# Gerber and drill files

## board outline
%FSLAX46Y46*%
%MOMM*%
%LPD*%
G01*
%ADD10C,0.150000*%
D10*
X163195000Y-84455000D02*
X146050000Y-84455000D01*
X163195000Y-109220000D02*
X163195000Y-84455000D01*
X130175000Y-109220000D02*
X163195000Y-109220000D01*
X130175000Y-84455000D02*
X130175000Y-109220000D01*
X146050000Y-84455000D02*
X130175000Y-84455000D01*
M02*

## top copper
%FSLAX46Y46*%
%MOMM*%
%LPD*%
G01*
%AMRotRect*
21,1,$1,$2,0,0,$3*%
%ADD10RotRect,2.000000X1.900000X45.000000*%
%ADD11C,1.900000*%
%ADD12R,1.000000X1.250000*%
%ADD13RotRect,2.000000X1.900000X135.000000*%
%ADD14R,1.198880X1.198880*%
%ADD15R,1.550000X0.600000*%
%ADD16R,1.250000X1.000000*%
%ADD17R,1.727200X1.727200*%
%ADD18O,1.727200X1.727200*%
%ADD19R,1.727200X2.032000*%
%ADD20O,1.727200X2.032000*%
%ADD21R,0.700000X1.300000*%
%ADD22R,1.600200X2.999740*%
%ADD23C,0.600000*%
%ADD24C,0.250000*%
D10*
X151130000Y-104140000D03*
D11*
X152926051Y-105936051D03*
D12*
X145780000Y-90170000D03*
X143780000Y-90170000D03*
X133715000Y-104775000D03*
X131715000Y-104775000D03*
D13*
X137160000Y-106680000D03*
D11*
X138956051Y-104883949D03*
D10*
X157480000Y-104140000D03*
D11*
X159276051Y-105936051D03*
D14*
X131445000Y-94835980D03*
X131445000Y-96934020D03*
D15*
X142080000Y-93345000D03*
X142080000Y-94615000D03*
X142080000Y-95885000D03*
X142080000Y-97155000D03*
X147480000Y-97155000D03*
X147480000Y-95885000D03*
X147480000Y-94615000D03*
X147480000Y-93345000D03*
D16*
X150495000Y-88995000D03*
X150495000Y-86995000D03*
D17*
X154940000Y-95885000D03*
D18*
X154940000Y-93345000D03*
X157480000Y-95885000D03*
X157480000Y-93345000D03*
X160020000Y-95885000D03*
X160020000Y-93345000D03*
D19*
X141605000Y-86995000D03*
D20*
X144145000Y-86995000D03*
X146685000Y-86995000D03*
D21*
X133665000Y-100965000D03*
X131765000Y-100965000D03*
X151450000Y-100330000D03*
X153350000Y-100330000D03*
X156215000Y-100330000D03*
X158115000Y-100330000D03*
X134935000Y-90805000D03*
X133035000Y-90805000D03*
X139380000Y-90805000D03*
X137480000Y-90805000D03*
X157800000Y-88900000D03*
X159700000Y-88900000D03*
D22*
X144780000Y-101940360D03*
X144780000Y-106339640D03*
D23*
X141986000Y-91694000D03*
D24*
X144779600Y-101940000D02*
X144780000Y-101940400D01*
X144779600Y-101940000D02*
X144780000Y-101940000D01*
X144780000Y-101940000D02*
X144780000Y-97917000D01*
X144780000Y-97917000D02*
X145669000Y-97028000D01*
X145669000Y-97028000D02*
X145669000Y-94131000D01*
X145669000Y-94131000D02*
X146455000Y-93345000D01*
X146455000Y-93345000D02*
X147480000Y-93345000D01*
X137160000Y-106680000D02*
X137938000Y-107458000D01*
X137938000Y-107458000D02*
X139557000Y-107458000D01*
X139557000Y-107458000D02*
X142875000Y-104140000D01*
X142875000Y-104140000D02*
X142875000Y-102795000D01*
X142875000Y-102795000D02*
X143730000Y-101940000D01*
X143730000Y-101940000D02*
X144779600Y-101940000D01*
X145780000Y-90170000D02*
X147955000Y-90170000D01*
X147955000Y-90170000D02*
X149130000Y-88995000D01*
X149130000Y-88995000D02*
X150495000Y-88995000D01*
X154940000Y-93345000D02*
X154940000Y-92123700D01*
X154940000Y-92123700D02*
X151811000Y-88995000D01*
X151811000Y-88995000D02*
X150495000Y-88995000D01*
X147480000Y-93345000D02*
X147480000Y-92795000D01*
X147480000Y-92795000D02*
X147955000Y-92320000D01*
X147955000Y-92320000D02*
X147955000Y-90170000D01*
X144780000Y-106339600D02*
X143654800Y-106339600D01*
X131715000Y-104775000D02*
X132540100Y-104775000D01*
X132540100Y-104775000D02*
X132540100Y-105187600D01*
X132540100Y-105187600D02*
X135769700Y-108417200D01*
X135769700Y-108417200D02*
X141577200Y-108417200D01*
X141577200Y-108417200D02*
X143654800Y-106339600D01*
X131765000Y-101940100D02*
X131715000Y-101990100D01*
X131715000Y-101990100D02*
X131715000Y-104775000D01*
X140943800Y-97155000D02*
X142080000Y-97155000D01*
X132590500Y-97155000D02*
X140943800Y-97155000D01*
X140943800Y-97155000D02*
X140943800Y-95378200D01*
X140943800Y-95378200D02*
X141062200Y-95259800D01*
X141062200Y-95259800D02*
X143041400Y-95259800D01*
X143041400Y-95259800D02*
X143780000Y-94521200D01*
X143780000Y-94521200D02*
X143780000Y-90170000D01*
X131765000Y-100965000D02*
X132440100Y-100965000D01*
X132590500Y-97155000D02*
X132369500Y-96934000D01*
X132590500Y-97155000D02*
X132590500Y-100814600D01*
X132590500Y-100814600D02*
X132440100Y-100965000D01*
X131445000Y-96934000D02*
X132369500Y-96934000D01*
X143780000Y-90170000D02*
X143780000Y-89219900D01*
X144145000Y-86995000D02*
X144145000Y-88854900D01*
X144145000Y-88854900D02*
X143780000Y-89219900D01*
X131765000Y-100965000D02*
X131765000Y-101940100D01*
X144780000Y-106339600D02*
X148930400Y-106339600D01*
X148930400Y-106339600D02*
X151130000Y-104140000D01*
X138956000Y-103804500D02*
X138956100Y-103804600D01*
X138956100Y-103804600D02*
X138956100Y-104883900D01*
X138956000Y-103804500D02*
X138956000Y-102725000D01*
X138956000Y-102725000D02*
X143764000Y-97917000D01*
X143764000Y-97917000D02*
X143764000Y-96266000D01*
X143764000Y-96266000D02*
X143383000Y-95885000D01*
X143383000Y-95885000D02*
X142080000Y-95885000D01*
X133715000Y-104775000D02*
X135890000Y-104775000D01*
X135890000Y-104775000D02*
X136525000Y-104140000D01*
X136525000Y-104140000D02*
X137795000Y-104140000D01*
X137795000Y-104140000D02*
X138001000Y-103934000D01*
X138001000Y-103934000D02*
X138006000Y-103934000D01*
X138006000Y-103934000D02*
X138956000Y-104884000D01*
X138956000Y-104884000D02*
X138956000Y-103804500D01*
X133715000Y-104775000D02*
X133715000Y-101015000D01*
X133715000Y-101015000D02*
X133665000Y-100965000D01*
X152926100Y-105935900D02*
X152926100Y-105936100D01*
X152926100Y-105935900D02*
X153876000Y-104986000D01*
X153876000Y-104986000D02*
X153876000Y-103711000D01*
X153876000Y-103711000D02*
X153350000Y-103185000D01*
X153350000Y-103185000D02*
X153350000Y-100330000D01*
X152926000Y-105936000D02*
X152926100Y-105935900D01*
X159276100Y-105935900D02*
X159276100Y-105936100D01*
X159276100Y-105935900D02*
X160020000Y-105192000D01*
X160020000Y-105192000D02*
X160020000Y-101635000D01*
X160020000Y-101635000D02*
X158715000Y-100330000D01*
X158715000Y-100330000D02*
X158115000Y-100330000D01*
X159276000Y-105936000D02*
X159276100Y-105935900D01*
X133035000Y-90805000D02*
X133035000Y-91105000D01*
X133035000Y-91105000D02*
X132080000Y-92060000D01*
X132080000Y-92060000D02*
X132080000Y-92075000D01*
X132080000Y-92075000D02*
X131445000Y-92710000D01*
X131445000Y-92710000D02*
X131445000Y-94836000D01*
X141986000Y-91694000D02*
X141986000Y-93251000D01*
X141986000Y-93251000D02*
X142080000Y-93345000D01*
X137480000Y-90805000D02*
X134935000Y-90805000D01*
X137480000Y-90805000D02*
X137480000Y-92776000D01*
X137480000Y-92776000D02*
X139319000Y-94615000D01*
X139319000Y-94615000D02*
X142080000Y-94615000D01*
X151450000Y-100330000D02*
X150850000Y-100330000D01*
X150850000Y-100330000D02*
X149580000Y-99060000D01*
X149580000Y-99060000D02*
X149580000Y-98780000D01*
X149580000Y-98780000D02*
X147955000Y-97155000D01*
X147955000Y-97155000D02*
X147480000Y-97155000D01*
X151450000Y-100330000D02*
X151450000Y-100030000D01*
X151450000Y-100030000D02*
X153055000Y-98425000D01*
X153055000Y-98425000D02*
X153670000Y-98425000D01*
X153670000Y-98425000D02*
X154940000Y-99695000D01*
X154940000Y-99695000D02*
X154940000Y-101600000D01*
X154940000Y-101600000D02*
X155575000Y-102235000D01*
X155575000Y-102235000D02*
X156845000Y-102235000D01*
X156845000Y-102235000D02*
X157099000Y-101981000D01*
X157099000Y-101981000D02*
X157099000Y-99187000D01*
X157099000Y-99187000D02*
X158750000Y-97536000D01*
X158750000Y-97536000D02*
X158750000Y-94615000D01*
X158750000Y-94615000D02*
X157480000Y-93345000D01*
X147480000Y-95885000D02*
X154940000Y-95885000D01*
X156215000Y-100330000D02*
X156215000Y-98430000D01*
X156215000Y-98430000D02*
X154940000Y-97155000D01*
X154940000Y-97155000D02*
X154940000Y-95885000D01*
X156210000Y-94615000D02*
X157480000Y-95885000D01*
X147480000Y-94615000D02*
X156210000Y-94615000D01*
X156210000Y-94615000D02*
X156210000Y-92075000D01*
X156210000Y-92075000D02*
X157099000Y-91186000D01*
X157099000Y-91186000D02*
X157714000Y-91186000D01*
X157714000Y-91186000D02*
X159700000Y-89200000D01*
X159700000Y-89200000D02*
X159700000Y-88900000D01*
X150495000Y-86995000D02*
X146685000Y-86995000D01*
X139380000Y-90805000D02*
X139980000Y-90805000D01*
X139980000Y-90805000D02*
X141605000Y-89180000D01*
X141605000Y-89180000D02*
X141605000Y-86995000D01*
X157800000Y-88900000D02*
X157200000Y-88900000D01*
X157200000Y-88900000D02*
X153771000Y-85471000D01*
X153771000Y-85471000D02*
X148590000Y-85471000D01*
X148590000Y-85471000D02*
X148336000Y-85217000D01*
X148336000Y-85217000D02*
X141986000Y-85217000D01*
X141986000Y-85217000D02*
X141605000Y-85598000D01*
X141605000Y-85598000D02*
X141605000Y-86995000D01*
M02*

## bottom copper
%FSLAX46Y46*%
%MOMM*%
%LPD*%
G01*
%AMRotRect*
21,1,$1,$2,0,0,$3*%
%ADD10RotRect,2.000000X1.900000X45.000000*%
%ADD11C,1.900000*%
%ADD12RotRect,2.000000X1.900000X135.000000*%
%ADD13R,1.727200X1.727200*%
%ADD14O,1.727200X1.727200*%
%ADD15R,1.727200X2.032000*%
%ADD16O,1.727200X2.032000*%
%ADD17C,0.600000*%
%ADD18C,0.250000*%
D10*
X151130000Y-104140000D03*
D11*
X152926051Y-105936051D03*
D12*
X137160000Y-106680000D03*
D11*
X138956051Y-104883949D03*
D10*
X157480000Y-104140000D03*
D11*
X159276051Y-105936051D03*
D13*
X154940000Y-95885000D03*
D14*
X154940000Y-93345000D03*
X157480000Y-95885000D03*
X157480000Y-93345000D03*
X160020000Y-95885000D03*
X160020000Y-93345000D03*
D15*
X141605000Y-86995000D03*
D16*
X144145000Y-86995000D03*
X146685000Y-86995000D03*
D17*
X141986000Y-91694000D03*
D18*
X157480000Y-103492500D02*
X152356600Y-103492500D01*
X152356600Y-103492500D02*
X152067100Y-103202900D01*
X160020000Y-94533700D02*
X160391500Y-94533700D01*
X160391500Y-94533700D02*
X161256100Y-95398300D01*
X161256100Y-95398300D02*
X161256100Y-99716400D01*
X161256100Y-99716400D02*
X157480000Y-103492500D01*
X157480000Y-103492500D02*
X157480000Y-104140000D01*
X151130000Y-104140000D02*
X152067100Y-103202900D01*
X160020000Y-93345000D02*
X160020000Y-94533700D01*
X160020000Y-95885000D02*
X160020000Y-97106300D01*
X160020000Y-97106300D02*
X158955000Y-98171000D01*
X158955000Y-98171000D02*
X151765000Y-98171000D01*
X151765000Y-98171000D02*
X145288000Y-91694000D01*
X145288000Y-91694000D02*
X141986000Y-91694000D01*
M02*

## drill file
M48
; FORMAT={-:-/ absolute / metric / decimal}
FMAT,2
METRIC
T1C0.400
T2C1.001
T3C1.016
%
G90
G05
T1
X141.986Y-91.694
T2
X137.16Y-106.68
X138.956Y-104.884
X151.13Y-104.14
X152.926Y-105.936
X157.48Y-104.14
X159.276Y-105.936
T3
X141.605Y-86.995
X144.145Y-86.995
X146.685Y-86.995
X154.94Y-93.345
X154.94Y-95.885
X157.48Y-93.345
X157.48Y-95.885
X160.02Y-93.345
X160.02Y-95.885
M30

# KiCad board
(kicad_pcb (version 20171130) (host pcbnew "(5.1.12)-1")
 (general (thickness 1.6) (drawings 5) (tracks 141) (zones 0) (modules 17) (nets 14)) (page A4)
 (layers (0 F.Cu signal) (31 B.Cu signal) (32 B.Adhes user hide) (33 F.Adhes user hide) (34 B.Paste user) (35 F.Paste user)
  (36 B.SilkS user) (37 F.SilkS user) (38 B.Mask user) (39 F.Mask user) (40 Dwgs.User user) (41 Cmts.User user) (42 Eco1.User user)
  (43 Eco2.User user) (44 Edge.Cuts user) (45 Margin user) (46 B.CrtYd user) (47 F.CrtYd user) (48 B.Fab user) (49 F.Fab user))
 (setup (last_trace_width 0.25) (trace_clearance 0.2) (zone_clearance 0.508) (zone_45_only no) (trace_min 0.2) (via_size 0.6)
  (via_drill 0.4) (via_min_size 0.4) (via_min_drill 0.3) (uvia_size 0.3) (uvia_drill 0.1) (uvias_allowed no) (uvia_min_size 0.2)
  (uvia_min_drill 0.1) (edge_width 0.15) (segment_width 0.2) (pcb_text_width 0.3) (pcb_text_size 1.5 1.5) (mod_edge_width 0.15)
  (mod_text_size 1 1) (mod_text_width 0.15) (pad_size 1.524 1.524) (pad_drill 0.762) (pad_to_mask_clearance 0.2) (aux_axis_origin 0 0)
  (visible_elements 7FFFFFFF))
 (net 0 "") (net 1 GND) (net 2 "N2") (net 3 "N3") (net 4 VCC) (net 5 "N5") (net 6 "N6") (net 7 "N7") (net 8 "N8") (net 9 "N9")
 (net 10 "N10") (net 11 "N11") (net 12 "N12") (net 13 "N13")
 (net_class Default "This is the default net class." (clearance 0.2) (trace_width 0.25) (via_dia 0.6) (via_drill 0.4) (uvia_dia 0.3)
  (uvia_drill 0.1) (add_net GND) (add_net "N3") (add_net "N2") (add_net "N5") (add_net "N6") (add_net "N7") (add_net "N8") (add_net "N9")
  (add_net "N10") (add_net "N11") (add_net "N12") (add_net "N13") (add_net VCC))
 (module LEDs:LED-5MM (layer F.Cu) (at 151.13 104.14 315)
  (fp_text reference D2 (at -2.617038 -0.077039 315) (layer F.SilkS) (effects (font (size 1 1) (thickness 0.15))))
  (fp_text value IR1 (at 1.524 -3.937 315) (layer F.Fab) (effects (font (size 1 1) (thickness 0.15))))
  (pad 1 thru_hole rect (at 0 0 45) (size 2 1.9) (drill 1.00076) (layers *.Cu *.Mask F.SilkS) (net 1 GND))
  (pad 2 thru_hole circle (at 2.54 0 315) (size 1.9 1.9) (drill 1.00076) (layers *.Cu *.Mask F.SilkS) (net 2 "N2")))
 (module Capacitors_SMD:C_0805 (layer F.Cu) (at 144.78 90.17 180)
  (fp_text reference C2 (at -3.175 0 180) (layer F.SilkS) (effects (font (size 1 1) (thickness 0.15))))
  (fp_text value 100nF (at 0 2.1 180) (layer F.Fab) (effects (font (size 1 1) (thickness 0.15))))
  (pad 1 smd rect (at -1 0 180) (size 1 1.25) (layers F.Cu F.Paste F.Mask) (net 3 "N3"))
  (pad 2 smd rect (at 1 0 180) (size 1 1.25) (layers F.Cu F.Paste F.Mask) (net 1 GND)))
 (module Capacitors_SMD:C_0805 (layer F.Cu) (at 132.715 104.775 180)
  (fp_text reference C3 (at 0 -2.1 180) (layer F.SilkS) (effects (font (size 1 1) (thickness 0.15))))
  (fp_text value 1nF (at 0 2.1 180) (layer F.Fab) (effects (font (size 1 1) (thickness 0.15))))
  (pad 1 smd rect (at -1 0 180) (size 1 1.25) (layers F.Cu F.Paste F.Mask) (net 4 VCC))
  (pad 2 smd rect (at 1 0 180) (size 1 1.25) (layers F.Cu F.Paste F.Mask) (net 1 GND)))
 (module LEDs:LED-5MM (layer F.Cu) (at 137.16 106.68 45)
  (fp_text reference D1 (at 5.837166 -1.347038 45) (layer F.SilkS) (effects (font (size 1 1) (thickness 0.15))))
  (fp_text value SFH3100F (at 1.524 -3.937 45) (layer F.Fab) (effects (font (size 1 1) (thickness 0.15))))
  (pad 1 thru_hole rect (at 0 0 135) (size 2 1.9) (drill 1.00076) (layers *.Cu *.Mask F.SilkS) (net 3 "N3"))
  (pad 2 thru_hole circle (at 2.54 0 45) (size 1.9 1.9) (drill 1.00076) (layers *.Cu *.Mask F.SilkS) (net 4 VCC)))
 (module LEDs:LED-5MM (layer F.Cu) (at 157.48 104.14 315)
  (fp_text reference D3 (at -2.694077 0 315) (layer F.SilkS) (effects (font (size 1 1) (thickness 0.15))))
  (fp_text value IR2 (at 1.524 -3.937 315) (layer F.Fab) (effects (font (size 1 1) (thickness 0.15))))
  (pad 1 thru_hole rect (at 0 0 45) (size 2 1.9) (drill 1.00076) (layers *.Cu *.Mask F.SilkS) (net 1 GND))
  (pad 2 thru_hole circle (at 2.54 0 315) (size 1.9 1.9) (drill 1.00076) (layers *.Cu *.Mask F.SilkS) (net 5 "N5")))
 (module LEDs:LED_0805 (layer F.Cu) (at 131.445 95.885 90)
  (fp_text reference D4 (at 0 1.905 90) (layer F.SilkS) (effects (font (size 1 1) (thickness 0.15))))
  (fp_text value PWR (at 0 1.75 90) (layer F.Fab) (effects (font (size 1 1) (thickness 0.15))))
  (pad 2 smd rect (at 1.04902 0 270) (size 1.19888 1.19888) (layers F.Cu F.Paste F.Mask) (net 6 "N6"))
  (pad 1 smd rect (at -1.04902 0 270) (size 1.19888 1.19888) (layers F.Cu F.Paste F.Mask) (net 1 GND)))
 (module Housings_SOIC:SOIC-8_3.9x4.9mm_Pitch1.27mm (layer F.Cu) (at 144.78 95.25)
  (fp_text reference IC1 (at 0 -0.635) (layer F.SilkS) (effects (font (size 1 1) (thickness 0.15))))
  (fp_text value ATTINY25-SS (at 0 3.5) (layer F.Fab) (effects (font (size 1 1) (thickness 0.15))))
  (pad 1 smd rect (at -2.7 -1.905) (size 1.55 0.6) (layers F.Cu F.Paste F.Mask) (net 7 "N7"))
  (pad 2 smd rect (at -2.7 -0.635) (size 1.55 0.6) (layers F.Cu F.Paste F.Mask) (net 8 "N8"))
  (pad 3 smd rect (at -2.7 0.635) (size 1.55 0.6) (layers F.Cu F.Paste F.Mask) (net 4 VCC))
  (pad 4 smd rect (at -2.7 1.905) (size 1.55 0.6) (layers F.Cu F.Paste F.Mask) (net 1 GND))
  (pad 5 smd rect (at 2.7 1.905) (size 1.55 0.6) (layers F.Cu F.Paste F.Mask) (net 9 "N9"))
  (pad 6 smd rect (at 2.7 0.635) (size 1.55 0.6) (layers F.Cu F.Paste F.Mask) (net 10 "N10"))
  (pad 7 smd rect (at 2.7 -0.635) (size 1.55 0.6) (layers F.Cu F.Paste F.Mask) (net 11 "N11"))
  (pad 8 smd rect (at 2.7 -1.905) (size 1.55 0.6) (layers F.Cu F.Paste F.Mask) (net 3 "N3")))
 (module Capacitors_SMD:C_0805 (layer F.Cu) (at 150.495 87.995 90)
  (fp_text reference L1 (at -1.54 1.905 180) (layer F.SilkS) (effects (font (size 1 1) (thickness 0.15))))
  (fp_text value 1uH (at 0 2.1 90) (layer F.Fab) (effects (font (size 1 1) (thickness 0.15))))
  (pad 1 smd rect (at -1 0 90) (size 1 1.25) (layers F.Cu F.Paste F.Mask) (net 3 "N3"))
  (pad 2 smd rect (at 1 0 90) (size 1 1.25) (layers F.Cu F.Paste F.Mask) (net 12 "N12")))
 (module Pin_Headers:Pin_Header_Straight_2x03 (layer F.Cu) (at 154.94 95.885 90)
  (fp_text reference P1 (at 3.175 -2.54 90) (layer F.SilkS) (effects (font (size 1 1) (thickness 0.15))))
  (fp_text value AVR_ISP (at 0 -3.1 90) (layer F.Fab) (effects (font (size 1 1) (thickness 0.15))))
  (pad 1 thru_hole rect (at 0 0 90) (size 1.7272 1.7272) (drill 1.016) (layers *.Cu *.Mask F.SilkS) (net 10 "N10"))
  (pad 2 thru_hole oval (at 2.54 0 90) (size 1.7272 1.7272) (drill 1.016) (layers *.Cu *.Mask F.SilkS) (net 3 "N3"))
  (pad 3 thru_hole oval (at 0 2.54 90) (size 1.7272 1.7272) (drill 1.016) (layers *.Cu *.Mask F.SilkS) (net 11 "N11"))
  (pad 4 thru_hole oval (at 2.54 2.54 90) (size 1.7272 1.7272) (drill 1.016) (layers *.Cu *.Mask F.SilkS) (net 9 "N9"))
  (pad 5 thru_hole oval (at 0 5.08 90) (size 1.7272 1.7272) (drill 1.016) (layers *.Cu *.Mask F.SilkS) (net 7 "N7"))
  (pad 6 thru_hole oval (at 2.54 5.08 90) (size 1.7272 1.7272) (drill 1.016) (layers *.Cu *.Mask F.SilkS) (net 1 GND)))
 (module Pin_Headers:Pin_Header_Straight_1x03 (layer F.Cu) (at 141.605 86.995 90)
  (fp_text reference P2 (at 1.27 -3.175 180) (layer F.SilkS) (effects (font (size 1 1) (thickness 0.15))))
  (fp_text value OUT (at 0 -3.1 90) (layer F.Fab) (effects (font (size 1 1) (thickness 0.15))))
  (pad 1 thru_hole rect (at 0 0 90) (size 2.032 1.7272) (drill 1.016) (layers *.Cu *.Mask F.SilkS) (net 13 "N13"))
  (pad 2 thru_hole oval (at 0 2.54 90) (size 2.032 1.7272) (drill 1.016) (layers *.Cu *.Mask F.SilkS) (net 1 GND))
  (pad 3 thru_hole oval (at 0 5.08 90) (size 2.032 1.7272) (drill 1.016) (layers *.Cu *.Mask F.SilkS) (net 12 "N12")))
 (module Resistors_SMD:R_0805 (layer F.Cu) (at 132.715 100.965 180)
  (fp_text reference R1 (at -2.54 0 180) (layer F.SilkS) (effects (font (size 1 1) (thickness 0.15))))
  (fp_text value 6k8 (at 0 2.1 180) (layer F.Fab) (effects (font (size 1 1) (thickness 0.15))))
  (pad 1 smd rect (at -0.95 0 180) (size 0.7 1.3) (layers F.Cu F.Paste F.Mask) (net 4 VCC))
  (pad 2 smd rect (at 0.95 0 180) (size 0.7 1.3) (layers F.Cu F.Paste F.Mask) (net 1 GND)))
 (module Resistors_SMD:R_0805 (layer F.Cu) (at 152.4 100.33)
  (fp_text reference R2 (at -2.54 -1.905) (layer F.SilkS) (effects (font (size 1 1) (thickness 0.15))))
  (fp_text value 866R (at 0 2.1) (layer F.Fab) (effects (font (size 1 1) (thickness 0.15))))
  (pad 1 smd rect (at -0.95 0) (size 0.7 1.3) (layers F.Cu F.Paste F.Mask) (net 9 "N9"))
  (pad 2 smd rect (at 0.95 0) (size 0.7 1.3) (layers F.Cu F.Paste F.Mask) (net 2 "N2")))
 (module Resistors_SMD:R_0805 (layer F.Cu) (at 157.165 100.33)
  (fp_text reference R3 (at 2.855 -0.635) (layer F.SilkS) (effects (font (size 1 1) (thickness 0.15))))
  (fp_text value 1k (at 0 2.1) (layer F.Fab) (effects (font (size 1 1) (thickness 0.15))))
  (pad 1 smd rect (at -0.95 0) (size 0.7 1.3) (layers F.Cu F.Paste F.Mask) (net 10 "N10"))
  (pad 2 smd rect (at 0.95 0) (size 0.7 1.3) (layers F.Cu F.Paste F.Mask) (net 5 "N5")))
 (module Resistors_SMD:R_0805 (layer F.Cu) (at 133.985 90.805 180)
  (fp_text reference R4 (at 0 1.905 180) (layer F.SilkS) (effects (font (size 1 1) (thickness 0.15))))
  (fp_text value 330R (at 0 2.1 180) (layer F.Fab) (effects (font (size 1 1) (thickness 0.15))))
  (pad 1 smd rect (at -0.95 0 180) (size 0.7 1.3) (layers F.Cu F.Paste F.Mask) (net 8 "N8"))
  (pad 2 smd rect (at 0.95 0 180) (size 0.7 1.3) (layers F.Cu F.Paste F.Mask) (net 6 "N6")))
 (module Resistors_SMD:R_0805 (layer F.Cu) (at 138.43 90.805 180)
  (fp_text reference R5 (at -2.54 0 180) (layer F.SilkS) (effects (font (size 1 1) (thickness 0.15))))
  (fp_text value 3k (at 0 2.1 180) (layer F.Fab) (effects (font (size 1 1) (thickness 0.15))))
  (pad 1 smd rect (at -0.95 0 180) (size 0.7 1.3) (layers F.Cu F.Paste F.Mask) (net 13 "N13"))
  (pad 2 smd rect (at 0.95 0 180) (size 0.7 1.3) (layers F.Cu F.Paste F.Mask) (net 8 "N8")))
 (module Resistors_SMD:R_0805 (layer F.Cu) (at 158.75 88.9)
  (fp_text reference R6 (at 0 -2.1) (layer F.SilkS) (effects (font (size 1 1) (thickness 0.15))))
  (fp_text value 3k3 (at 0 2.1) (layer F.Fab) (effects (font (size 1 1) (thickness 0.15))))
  (pad 1 smd rect (at -0.95 0) (size 0.7 1.3) (layers F.Cu F.Paste F.Mask) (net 13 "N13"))
  (pad 2 smd rect (at 0.95 0) (size 0.7 1.3) (layers F.Cu F.Paste F.Mask) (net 11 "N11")))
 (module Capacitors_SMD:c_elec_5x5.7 (layer F.Cu) (at 144.78 104.14 90)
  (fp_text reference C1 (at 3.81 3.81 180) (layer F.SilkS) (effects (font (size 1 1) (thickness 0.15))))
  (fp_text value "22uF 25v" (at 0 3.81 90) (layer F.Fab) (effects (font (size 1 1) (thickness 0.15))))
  (pad 1 smd rect (at 2.19964 0 90) (size 2.99974 1.6002) (layers F.Cu F.Paste F.Mask) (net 3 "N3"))
  (pad 2 smd rect (at -2.19964 0 90) (size 2.99974 1.6002) (layers F.Cu F.Paste F.Mask) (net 1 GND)))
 (gr_line (start 163.195 84.455) (end 146.05 84.455) (layer Edge.Cuts) (width 0.15))
 (gr_line (start 163.195 109.22) (end 163.195 84.455) (layer Edge.Cuts) (width 0.15))
 (gr_line (start 130.175 109.22) (end 163.195 109.22) (layer Edge.Cuts) (width 0.15))
 (gr_line (start 130.175 84.455) (end 130.175 109.22) (layer Edge.Cuts) (width 0.15))
 (gr_line (start 146.05 84.455) (end 130.175 84.455) (layer Edge.Cuts) (width 0.15))
 (segment (start 144.7796 101.94) (end 144.78 101.9404) (width 0.25) (layer F.Cu) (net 3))
 (segment (start 144.7796 101.94) (end 144.78 101.94) (width 0.25) (layer F.Cu) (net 3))
 (segment (start 144.78 101.94) (end 144.78 97.917) (width 0.25) (layer F.Cu) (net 3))
 (segment (start 144.78 97.917) (end 145.669 97.028) (width 0.25) (layer F.Cu) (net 3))
 (segment (start 145.669 97.028) (end 145.669 94.131) (width 0.25) (layer F.Cu) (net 3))
 (segment (start 145.669 94.131) (end 146.455 93.345) (width 0.25) (layer F.Cu) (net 3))
 (segment (start 146.455 93.345) (end 147.48 93.345) (width 0.25) (layer F.Cu) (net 3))
 (segment (start 137.16 106.68) (end 137.938 107.458) (width 0.25) (layer F.Cu) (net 3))
 (segment (start 137.938 107.458) (end 139.557 107.458) (width 0.25) (layer F.Cu) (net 3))
 (segment (start 139.557 107.458) (end 142.875 104.14) (width 0.25) (layer F.Cu) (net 3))
 (segment (start 142.875 104.14) (end 142.875 102.795) (width 0.25) (layer F.Cu) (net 3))
 (segment (start 142.875 102.795) (end 143.73 101.94) (width 0.25) (layer F.Cu) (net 3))
 (segment (start 143.73 101.94) (end 144.7796 101.94) (width 0.25) (layer F.Cu) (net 3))
 (segment (start 145.78 90.17) (end 147.955 90.17) (width 0.25) (layer F.Cu) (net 3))
 (segment (start 147.955 90.17) (end 149.13 88.995) (width 0.25) (layer F.Cu) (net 3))
 (segment (start 149.13 88.995) (end 150.495 88.995) (width 0.25) (layer F.Cu) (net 3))
 (segment (start 154.94 93.345) (end 154.94 92.1237) (width 0.25) (layer F.Cu) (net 3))
 (segment (start 154.94 92.1237) (end 151.811 88.995) (width 0.25) (layer F.Cu) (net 3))
 (segment (start 151.811 88.995) (end 150.495 88.995) (width 0.25) (layer F.Cu) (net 3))
 (segment (start 147.48 93.345) (end 147.48 92.795) (width 0.25) (layer F.Cu) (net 3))
 (segment (start 147.48 92.795) (end 147.955 92.32) (width 0.25) (layer F.Cu) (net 3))
 (segment (start 147.955 92.32) (end 147.955 90.17) (width 0.25) (layer F.Cu) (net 3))
 (segment (start 157.48 103.4925) (end 152.3566 103.4925) (width 0.25) (layer B.Cu) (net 1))
 (segment (start 152.3566 103.4925) (end 152.0671 103.2029) (width 0.25) (layer B.Cu) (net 1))
 (segment (start 160.02 94.5337) (end 160.3915 94.5337) (width 0.25) (layer B.Cu) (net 1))
 (segment (start 160.3915 94.5337) (end 161.2561 95.3983) (width 0.25) (layer B.Cu) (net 1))
 (segment (start 161.2561 95.3983) (end 161.2561 99.7164) (width 0.25) (layer B.Cu) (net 1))
 (segment (start 161.2561 99.7164) (end 157.48 103.4925) (width 0.25) (layer B.Cu) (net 1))
 (segment (start 157.48 103.4925) (end 157.48 104.14) (width 0.25) (layer B.Cu) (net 1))
 (segment (start 151.13 104.14) (end 152.0671 103.2029) (width 0.25) (layer B.Cu) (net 1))
 (segment (start 144.78 106.3396) (end 143.6548 106.3396) (width 0.25) (layer F.Cu) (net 1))
 (segment (start 131.715 104.775) (end 132.5401 104.775) (width 0.25) (layer F.Cu) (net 1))
 (segment (start 132.5401 104.775) (end 132.5401 105.1876) (width 0.25) (layer F.Cu) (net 1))
 (segment (start 132.5401 105.1876) (end 135.7697 108.4172) (width 0.25) (layer F.Cu) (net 1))
 (segment (start 135.7697 108.4172) (end 141.5772 108.4172) (width 0.25) (layer F.Cu) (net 1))
 (segment (start 141.5772 108.4172) (end 143.6548 106.3396) (width 0.25) (layer F.Cu) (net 1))
 (segment (start 131.765 101.9401) (end 131.715 101.9901) (width 0.25) (layer F.Cu) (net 1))
 (segment (start 131.715 101.9901) (end 131.715 104.775) (width 0.25) (layer F.Cu) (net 1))
 (segment (start 140.9438 97.155) (end 142.08 97.155) (width 0.25) (layer F.Cu) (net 1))
 (segment (start 132.5905 97.155) (end 140.9438 97.155) (width 0.25) (layer F.Cu) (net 1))
 (segment (start 140.9438 97.155) (end 140.9438 95.3782) (width 0.25) (layer F.Cu) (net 1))
 (segment (start 140.9438 95.3782) (end 141.0622 95.2598) (width 0.25) (layer F.Cu) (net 1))
 (segment (start 141.0622 95.2598) (end 143.0414 95.2598) (width 0.25) (layer F.Cu) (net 1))
 (segment (start 143.0414 95.2598) (end 143.78 94.5212) (width 0.25) (layer F.Cu) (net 1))
 (segment (start 143.78 94.5212) (end 143.78 90.17) (width 0.25) (layer F.Cu) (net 1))
 (segment (start 131.765 100.965) (end 132.4401 100.965) (width 0.25) (layer F.Cu) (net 1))
 (segment (start 132.5905 97.155) (end 132.3695 96.934) (width 0.25) (layer F.Cu) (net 1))
 (segment (start 132.5905 97.155) (end 132.5905 100.8146) (width 0.25) (layer F.Cu) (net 1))
 (segment (start 132.5905 100.8146) (end 132.4401 100.965) (width 0.25) (layer F.Cu) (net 1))
 (segment (start 131.445 96.934) (end 132.3695 96.934) (width 0.25) (layer F.Cu) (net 1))
 (segment (start 160.02 93.345) (end 160.02 94.5337) (width 0.25) (layer B.Cu) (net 1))
 (segment (start 143.78 90.17) (end 143.78 89.2199) (width 0.25) (layer F.Cu) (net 1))
 (segment (start 144.145 86.995) (end 144.145 88.8549) (width 0.25) (layer F.Cu) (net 1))
 (segment (start 144.145 88.8549) (end 143.78 89.2199) (width 0.25) (layer F.Cu) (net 1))
 (segment (start 131.765 100.965) (end 131.765 101.9401) (width 0.25) (layer F.Cu) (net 1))
 (segment (start 144.78 106.3396) (end 148.9304 106.3396) (width 0.25) (layer F.Cu) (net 1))
 (segment (start 148.9304 106.3396) (end 151.13 104.14) (width 0.25) (layer F.Cu) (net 1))
 (segment (start 138.956 103.8045) (end 138.9561 103.8046) (width 0.25) (layer F.Cu) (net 4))
 (segment (start 138.9561 103.8046) (end 138.9561 104.8839) (width 0.25) (layer F.Cu) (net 4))
 (segment (start 138.956 103.8045) (end 138.956 102.725) (width 0.25) (layer F.Cu) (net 4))
 (segment (start 138.956 102.725) (end 143.764 97.917) (width 0.25) (layer F.Cu) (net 4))
 (segment (start 143.764 97.917) (end 143.764 96.266) (width 0.25) (layer F.Cu) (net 4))
 (segment (start 143.764 96.266) (end 143.383 95.885) (width 0.25) (layer F.Cu) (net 4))
 (segment (start 143.383 95.885) (end 142.08 95.885) (width 0.25) (layer F.Cu) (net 4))
 (segment (start 133.715 104.775) (end 135.89 104.775) (width 0.25) (layer F.Cu) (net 4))
 (segment (start 135.89 104.775) (end 136.525 104.14) (width 0.25) (layer F.Cu) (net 4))
 (segment (start 136.525 104.14) (end 137.795 104.14) (width 0.25) (layer F.Cu) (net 4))
 (segment (start 137.795 104.14) (end 138.001 103.934) (width 0.25) (layer F.Cu) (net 4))
 (segment (start 138.001 103.934) (end 138.006 103.934) (width 0.25) (layer F.Cu) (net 4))
 (segment (start 138.006 103.934) (end 138.956 104.884) (width 0.25) (layer F.Cu) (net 4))
 (segment (start 138.956 104.884) (end 138.956 103.8045) (width 0.25) (layer F.Cu) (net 4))
 (segment (start 133.715 104.775) (end 133.715 101.015) (width 0.25) (layer F.Cu) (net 4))
 (segment (start 133.715 101.015) (end 133.665 100.965) (width 0.25) (layer F.Cu) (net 4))
 (segment (start 152.9261 105.9359) (end 152.9261 105.9361) (width 0.25) (layer F.Cu) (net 2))
 (segment (start 152.9261 105.9359) (end 153.876 104.986) (width 0.25) (layer F.Cu) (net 2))
 (segment (start 153.876 104.986) (end 153.876 103.711) (width 0.25) (layer F.Cu) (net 2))
 (segment (start 153.876 103.711) (end 153.35 103.185) (width 0.25) (layer F.Cu) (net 2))
 (segment (start 153.35 103.185) (end 153.35 100.33) (width 0.25) (layer F.Cu) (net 2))
 (segment (start 152.926 105.936) (end 152.9261 105.9359) (width 0.25) (layer F.Cu) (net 2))
 (segment (start 159.2761 105.9359) (end 159.2761 105.9361) (width 0.25) (layer F.Cu) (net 5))
 (segment (start 159.2761 105.9359) (end 160.02 105.192) (width 0.25) (layer F.Cu) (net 5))
 (segment (start 160.02 105.192) (end 160.02 101.635) (width 0.25) (layer F.Cu) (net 5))
 (segment (start 160.02 101.635) (end 158.715 100.33) (width 0.25) (layer F.Cu) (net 5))
 (segment (start 158.715 100.33) (end 158.115 100.33) (width 0.25) (layer F.Cu) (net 5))
 (segment (start 159.276 105.936) (end 159.2761 105.9359) (width 0.25) (layer F.Cu) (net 5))
 (segment (start 133.035 90.805) (end 133.035 91.105) (width 0.25) (layer F.Cu) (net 6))
 (segment (start 133.035 91.105) (end 132.08 92.06) (width 0.25) (layer F.Cu) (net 6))
 (segment (start 132.08 92.06) (end 132.08 92.075) (width 0.25) (layer F.Cu) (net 6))
 (segment (start 132.08 92.075) (end 131.445 92.71) (width 0.25) (layer F.Cu) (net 6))
 (segment (start 131.445 92.71) (end 131.445 94.836) (width 0.25) (layer F.Cu) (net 6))
 (segment (start 160.02 95.885) (end 160.02 97.1063) (width 0.25) (layer B.Cu) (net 7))
 (segment (start 160.02 97.1063) (end 158.955 98.171) (width 0.25) (layer B.Cu) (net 7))
 (segment (start 158.955 98.171) (end 151.765 98.171) (width 0.25) (layer B.Cu) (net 7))
 (segment (start 151.765 98.171) (end 145.288 91.694) (width 0.25) (layer B.Cu) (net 7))
 (segment (start 145.288 91.694) (end 141.986 91.694) (width 0.25) (layer B.Cu) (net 7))
 (segment (start 141.986 91.694) (end 141.986 93.251) (width 0.25) (layer F.Cu) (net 7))
 (segment (start 141.986 93.251) (end 142.08 93.345) (width 0.25) (layer F.Cu) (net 7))
 (via (at 141.986 91.694) (size 0.6) (layers F.Cu B.Cu) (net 7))
 (segment (start 137.48 90.805) (end 134.935 90.805) (width 0.25) (layer F.Cu) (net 8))
 (segment (start 137.48 90.805) (end 137.48 92.776) (width 0.25) (layer F.Cu) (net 8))
 (segment (start 137.48 92.776) (end 139.319 94.615) (width 0.25) (layer F.Cu) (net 8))
 (segment (start 139.319 94.615) (end 142.08 94.615) (width 0.25) (layer F.Cu) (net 8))
 (segment (start 151.45 100.33) (end 150.85 100.33) (width 0.25) (layer F.Cu) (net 9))
 (segment (start 150.85 100.33) (end 149.58 99.06) (width 0.25) (layer F.Cu) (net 9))
 (segment (start 149.58 99.06) (end 149.58 98.78) (width 0.25) (layer F.Cu) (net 9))
 (segment (start 149.58 98.78) (end 147.955 97.155) (width 0.25) (layer F.Cu) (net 9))
 (segment (start 147.955 97.155) (end 147.48 97.155) (width 0.25) (layer F.Cu) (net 9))
 (segment (start 151.45 100.33) (end 151.45 100.03) (width 0.25) (layer F.Cu) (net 9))
 (segment (start 151.45 100.03) (end 153.055 98.425) (width 0.25) (layer F.Cu) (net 9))
 (segment (start 153.055 98.425) (end 153.67 98.425) (width 0.25) (layer F.Cu) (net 9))
 (segment (start 153.67 98.425) (end 154.94 99.695) (width 0.25) (layer F.Cu) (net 9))
 (segment (start 154.94 99.695) (end 154.94 101.6) (width 0.25) (layer F.Cu) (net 9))
 (segment (start 154.94 101.6) (end 155.575 102.235) (width 0.25) (layer F.Cu) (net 9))
 (segment (start 155.575 102.235) (end 156.845 102.235) (width 0.25) (layer F.Cu) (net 9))
 (segment (start 156.845 102.235) (end 157.099 101.981) (width 0.25) (layer F.Cu) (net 9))
 (segment (start 157.099 101.981) (end 157.099 99.187) (width 0.25) (layer F.Cu) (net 9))
 (segment (start 157.099 99.187) (end 158.75 97.536) (width 0.25) (layer F.Cu) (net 9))
 (segment (start 158.75 97.536) (end 158.75 94.615) (width 0.25) (layer F.Cu) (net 9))
 (segment (start 158.75 94.615) (end 157.48 93.345) (width 0.25) (layer F.Cu) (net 9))
 (segment (start 147.48 95.885) (end 154.94 95.885) (width 0.25) (layer F.Cu) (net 10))
 (segment (start 156.215 100.33) (end 156.215 98.43) (width 0.25) (layer F.Cu) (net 10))
 (segment (start 156.215 98.43) (end 154.94 97.155) (width 0.25) (layer F.Cu) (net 10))
 (segment (start 154.94 97.155) (end 154.94 95.885) (width 0.25) (layer F.Cu) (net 10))
 (segment (start 156.21 94.615) (end 157.48 95.885) (width 0.25) (layer F.Cu) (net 11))
 (segment (start 147.48 94.615) (end 156.21 94.615) (width 0.25) (layer F.Cu) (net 11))
 (segment (start 156.21 94.615) (end 156.21 92.075) (width 0.25) (layer F.Cu) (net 11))
 (segment (start 156.21 92.075) (end 157.099 91.186) (width 0.25) (layer F.Cu) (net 11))
 (segment (start 157.099 91.186) (end 157.714 91.186) (width 0.25) (layer F.Cu) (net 11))
 (segment (start 157.714 91.186) (end 159.7 89.2) (width 0.25) (layer F.Cu) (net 11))
 (segment (start 159.7 89.2) (end 159.7 88.9) (width 0.25) (layer F.Cu) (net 11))
 (segment (start 150.495 86.995) (end 146.685 86.995) (width 0.25) (layer F.Cu) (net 12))
 (segment (start 139.38 90.805) (end 139.98 90.805) (width 0.25) (layer F.Cu) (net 13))
 (segment (start 139.98 90.805) (end 141.605 89.18) (width 0.25) (layer F.Cu) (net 13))
 (segment (start 141.605 89.18) (end 141.605 86.995) (width 0.25) (layer F.Cu) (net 13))
 (segment (start 157.8 88.9) (end 157.2 88.9) (width 0.25) (layer F.Cu) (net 13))
 (segment (start 157.2 88.9) (end 153.771 85.471) (width 0.25) (layer F.Cu) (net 13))
 (segment (start 153.771 85.471) (end 148.59 85.471) (width 0.25) (layer F.Cu) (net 13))
 (segment (start 148.59 85.471) (end 148.336 85.217) (width 0.25) (layer F.Cu) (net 13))
 (segment (start 148.336 85.217) (end 141.986 85.217) (width 0.25) (layer F.Cu) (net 13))
 (segment (start 141.986 85.217) (end 141.605 85.598) (width 0.25) (layer F.Cu) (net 13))
 (segment (start 141.605 85.598) (end 141.605 86.995) (width 0.25) (layer F.Cu) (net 13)))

